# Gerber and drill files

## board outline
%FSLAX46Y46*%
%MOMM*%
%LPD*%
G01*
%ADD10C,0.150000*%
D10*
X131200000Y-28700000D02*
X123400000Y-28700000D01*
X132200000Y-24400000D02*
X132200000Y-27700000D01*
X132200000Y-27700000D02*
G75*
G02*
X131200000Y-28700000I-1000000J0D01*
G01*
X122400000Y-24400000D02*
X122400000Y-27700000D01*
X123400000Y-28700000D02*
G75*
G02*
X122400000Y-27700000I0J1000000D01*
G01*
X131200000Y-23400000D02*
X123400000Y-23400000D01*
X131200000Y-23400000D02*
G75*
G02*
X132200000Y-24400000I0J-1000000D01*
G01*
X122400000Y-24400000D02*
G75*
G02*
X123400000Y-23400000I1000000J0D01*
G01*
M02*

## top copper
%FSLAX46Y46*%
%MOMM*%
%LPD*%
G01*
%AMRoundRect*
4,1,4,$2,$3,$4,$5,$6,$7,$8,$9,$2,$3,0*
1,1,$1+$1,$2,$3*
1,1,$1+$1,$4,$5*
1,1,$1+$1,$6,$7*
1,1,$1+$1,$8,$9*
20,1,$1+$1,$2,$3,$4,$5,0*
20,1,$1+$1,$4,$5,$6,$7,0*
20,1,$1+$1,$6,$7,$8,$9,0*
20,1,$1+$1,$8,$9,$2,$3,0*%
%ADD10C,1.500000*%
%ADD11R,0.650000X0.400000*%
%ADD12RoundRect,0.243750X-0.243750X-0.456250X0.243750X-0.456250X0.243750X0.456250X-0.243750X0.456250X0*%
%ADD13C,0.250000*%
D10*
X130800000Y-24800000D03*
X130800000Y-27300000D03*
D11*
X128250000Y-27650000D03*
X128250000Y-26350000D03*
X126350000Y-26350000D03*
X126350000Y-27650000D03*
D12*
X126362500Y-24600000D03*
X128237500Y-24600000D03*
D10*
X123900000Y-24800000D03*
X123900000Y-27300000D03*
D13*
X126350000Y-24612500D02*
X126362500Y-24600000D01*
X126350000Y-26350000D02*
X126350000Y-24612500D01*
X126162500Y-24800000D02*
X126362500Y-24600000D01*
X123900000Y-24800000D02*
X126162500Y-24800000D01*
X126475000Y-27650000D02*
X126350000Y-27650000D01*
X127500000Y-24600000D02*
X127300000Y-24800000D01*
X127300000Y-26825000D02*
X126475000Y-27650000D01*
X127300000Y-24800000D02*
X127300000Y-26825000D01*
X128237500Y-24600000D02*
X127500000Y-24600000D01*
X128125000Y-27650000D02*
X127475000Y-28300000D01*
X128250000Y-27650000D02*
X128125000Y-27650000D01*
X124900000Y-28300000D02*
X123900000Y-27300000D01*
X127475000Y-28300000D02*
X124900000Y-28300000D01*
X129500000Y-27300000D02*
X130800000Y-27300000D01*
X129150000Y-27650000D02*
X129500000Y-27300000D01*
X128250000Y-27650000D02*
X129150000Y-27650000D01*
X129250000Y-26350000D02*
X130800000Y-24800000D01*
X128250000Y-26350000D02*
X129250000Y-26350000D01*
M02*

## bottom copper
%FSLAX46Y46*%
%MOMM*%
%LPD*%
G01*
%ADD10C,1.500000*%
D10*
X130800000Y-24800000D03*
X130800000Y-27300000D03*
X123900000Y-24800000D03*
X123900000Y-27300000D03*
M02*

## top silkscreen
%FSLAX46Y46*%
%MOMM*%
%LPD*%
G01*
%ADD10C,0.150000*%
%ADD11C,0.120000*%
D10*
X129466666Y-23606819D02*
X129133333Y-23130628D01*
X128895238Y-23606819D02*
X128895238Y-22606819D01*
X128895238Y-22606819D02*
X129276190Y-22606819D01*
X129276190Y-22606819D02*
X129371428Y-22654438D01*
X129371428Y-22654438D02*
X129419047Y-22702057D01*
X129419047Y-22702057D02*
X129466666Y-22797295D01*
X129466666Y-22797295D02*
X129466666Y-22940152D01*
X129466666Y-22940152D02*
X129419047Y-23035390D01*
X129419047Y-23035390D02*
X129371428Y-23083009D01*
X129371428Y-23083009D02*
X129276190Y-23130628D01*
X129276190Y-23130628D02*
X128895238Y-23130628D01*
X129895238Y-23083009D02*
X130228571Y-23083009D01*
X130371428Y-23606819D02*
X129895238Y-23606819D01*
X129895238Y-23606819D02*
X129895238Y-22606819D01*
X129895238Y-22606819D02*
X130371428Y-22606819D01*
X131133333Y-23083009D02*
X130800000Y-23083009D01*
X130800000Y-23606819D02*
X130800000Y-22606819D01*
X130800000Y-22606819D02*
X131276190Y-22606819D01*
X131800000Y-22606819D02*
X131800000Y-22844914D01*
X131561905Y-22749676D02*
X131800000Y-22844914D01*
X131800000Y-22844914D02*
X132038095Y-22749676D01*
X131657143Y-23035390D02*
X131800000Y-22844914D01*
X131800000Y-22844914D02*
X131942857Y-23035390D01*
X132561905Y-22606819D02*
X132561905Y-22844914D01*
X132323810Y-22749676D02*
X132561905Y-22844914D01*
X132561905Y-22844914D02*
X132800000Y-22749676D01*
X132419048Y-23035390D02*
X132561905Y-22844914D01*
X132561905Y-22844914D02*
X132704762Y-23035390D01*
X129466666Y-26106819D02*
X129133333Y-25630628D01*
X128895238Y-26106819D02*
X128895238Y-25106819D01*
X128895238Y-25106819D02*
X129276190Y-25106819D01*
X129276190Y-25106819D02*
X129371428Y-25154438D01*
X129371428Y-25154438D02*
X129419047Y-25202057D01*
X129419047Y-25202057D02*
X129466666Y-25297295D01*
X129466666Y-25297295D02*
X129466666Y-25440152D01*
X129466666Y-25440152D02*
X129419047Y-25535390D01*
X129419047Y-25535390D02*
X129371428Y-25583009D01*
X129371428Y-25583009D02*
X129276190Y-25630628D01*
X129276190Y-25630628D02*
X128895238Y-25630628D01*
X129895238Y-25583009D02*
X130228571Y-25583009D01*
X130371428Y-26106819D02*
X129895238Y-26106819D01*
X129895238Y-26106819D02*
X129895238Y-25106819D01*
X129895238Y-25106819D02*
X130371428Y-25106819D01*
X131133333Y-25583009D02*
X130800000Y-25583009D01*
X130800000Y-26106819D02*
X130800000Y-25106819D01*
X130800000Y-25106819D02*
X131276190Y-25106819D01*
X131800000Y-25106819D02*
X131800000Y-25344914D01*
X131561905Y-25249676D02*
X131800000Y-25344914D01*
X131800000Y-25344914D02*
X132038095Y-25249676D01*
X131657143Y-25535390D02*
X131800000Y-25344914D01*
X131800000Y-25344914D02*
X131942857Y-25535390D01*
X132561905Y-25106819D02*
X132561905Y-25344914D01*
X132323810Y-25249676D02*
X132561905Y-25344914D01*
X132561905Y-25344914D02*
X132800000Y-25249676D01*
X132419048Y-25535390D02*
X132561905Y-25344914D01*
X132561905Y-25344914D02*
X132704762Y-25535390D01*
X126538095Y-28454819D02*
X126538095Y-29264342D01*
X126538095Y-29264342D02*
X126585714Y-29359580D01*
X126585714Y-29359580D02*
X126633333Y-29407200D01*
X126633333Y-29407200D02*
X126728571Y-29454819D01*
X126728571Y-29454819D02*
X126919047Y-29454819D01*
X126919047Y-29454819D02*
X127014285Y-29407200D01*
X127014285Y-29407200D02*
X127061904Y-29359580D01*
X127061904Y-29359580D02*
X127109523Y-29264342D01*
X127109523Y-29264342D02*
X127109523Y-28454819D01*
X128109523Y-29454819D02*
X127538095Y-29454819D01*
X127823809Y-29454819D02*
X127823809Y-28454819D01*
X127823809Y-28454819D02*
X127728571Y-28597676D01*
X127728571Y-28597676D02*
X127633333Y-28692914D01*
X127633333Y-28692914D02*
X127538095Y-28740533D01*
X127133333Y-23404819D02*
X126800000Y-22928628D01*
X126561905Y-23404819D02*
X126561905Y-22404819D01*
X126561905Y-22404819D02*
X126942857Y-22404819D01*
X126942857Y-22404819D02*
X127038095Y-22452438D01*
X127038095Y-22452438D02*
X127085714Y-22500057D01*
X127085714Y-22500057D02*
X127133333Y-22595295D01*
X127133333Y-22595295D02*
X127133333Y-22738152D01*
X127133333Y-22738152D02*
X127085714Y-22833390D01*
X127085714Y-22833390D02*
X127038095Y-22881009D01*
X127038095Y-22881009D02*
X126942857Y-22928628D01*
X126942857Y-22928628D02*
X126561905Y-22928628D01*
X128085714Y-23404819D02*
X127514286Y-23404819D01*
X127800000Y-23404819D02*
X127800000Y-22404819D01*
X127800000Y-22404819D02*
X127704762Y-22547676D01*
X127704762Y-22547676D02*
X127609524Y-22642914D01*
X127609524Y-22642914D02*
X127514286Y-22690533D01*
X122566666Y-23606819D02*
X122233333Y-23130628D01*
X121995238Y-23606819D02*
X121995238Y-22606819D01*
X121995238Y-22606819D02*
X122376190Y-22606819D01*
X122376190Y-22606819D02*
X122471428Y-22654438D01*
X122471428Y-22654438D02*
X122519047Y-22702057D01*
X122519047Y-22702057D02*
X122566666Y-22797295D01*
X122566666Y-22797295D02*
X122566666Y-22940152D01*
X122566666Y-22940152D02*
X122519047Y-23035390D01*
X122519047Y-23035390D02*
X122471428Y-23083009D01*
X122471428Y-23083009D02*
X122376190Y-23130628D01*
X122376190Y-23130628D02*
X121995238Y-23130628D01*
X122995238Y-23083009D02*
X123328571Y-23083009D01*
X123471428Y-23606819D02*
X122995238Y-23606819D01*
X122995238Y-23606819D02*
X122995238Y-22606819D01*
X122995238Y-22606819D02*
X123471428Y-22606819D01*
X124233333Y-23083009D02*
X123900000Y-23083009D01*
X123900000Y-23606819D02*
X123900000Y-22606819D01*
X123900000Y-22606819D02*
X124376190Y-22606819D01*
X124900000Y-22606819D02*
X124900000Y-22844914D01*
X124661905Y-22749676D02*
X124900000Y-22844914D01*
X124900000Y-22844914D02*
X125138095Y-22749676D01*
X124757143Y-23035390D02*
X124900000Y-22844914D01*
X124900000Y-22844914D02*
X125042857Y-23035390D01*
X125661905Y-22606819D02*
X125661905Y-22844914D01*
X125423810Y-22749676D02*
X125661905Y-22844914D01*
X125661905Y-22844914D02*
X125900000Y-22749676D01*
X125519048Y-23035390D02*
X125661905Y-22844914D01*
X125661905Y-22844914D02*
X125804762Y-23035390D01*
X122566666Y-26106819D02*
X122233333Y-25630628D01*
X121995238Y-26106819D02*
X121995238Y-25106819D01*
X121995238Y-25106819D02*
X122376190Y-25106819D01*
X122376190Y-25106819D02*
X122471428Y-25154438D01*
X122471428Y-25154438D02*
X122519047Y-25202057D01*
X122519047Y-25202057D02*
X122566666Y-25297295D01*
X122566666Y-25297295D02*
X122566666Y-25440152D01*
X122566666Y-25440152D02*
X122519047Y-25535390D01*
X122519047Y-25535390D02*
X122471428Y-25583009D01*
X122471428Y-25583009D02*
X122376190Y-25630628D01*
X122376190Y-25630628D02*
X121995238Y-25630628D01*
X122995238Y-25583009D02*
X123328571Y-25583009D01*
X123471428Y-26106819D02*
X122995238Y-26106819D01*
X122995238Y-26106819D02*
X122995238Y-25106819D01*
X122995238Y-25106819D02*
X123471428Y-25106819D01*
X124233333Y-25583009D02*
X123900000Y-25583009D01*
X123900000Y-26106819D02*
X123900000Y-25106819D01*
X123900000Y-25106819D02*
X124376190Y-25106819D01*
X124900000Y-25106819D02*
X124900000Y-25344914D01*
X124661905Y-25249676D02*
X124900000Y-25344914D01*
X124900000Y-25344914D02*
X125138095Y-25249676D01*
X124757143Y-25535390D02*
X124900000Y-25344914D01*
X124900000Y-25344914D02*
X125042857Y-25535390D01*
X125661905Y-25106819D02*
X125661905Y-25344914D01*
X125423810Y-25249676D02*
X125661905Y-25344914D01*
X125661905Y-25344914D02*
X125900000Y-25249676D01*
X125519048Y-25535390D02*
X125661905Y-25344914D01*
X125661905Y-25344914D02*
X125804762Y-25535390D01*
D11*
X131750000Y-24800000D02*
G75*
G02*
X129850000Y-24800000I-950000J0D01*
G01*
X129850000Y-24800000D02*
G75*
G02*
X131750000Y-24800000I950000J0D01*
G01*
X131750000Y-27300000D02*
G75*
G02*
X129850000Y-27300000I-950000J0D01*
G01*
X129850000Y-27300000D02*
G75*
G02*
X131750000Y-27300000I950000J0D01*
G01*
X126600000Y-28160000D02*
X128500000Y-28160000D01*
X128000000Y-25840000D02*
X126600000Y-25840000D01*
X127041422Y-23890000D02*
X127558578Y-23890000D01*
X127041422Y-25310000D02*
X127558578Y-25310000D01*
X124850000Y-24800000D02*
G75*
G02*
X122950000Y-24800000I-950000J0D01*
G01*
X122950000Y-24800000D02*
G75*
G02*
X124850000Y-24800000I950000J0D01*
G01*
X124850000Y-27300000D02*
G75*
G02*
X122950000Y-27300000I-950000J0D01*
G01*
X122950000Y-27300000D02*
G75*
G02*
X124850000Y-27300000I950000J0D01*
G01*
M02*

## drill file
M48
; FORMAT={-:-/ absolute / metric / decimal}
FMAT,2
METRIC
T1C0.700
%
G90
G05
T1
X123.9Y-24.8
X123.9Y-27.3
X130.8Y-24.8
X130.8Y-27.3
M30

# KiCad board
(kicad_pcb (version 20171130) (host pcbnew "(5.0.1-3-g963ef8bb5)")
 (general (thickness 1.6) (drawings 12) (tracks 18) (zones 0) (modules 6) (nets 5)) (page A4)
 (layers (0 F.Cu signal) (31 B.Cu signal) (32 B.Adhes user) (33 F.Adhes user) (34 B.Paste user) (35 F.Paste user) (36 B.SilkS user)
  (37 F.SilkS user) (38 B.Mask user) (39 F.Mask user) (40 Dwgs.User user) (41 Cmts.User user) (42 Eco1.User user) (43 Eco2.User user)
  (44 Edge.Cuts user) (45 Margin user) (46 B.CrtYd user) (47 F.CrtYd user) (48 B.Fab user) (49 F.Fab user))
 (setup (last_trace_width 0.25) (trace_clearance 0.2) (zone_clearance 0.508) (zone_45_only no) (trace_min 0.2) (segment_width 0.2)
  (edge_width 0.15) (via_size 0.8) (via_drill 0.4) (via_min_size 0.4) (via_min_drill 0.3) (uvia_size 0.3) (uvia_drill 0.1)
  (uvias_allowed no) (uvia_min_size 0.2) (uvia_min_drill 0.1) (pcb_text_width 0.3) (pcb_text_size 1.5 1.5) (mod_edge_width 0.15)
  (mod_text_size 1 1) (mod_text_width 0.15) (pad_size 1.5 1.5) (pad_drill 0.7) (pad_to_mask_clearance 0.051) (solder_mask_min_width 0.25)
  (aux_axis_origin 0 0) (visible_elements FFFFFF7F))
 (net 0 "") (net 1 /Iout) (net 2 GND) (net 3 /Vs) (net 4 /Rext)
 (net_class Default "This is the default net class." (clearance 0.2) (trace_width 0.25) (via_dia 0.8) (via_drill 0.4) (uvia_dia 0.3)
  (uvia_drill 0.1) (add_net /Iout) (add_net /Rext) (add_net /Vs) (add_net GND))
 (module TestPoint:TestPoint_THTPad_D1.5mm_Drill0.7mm (layer F.Cu) (at 130.8 24.8)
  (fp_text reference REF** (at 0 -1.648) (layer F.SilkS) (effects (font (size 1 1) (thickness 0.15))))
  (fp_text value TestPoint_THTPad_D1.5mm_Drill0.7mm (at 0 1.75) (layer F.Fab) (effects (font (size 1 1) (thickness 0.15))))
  (fp_circle (center 0 0) (end 0 0.95) (layer F.SilkS) (width 0.12))
  (pad 1 thru_hole circle (at 0 0) (size 1.5 1.5) (drill 0.7) (layers *.Cu *.Mask) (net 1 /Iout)))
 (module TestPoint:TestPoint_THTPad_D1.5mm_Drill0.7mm (layer F.Cu) (at 130.8 27.3)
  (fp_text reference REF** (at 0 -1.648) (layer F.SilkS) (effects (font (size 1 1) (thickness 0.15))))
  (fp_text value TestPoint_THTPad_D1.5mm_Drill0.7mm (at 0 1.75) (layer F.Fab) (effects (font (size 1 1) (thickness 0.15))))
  (fp_circle (center 0 0) (end 0 0.95) (layer F.SilkS) (width 0.12))
  (pad 1 thru_hole circle (at 0 0) (size 1.5 1.5) (drill 0.7) (layers *.Cu *.Mask) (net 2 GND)))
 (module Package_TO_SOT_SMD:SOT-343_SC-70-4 (layer F.Cu) (at 127.3 27 180)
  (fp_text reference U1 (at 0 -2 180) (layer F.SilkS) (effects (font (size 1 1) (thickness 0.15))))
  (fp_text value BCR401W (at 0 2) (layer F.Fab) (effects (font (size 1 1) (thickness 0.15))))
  (fp_line (start 0.7 -1.16) (end -1.2 -1.16) (layer F.SilkS) (width 0.12))
  (fp_line (start -0.7 1.16) (end 0.7 1.16) (layer F.SilkS) (width 0.12))
  (pad 1 smd rect (at -0.95 -0.65 180) (size 0.65 0.4) (layers F.Cu F.Paste F.Mask) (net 2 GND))
  (pad 2 smd rect (at -0.95 0.65 180) (size 0.65 0.4) (layers F.Cu F.Paste F.Mask) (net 1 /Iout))
  (pad 3 smd rect (at 0.95 0.65 180) (size 0.65 0.4) (layers F.Cu F.Paste F.Mask) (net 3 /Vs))
  (pad 4 smd rect (at 0.95 -0.65 180) (size 0.65 0.4) (layers F.Cu F.Paste F.Mask) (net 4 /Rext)))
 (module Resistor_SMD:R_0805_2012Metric (layer F.Cu) (at 127.3 24.6)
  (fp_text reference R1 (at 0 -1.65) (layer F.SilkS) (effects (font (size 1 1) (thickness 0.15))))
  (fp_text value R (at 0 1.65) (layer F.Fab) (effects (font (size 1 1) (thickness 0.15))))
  (fp_line (start -0.258578 -0.71) (end 0.258578 -0.71) (layer F.SilkS) (width 0.12))
  (fp_line (start -0.258578 0.71) (end 0.258578 0.71) (layer F.SilkS) (width 0.12))
  (pad 1 smd roundrect (at -0.9375 0) (size 0.975 1.4) (layers F.Cu F.Paste F.Mask) (roundrect_rratio 0.25) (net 3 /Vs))
  (pad 2 smd roundrect (at 0.9375 0) (size 0.975 1.4) (layers F.Cu F.Paste F.Mask) (roundrect_rratio 0.25) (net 4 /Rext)))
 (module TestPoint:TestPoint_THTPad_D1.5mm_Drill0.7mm (layer F.Cu) (at 123.9 24.8)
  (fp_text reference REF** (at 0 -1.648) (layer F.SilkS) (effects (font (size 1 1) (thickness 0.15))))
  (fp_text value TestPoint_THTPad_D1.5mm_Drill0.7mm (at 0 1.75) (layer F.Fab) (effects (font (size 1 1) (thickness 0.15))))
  (fp_circle (center 0 0) (end 0 0.95) (layer F.SilkS) (width 0.12))
  (pad 1 thru_hole circle (at 0 0) (size 1.5 1.5) (drill 0.7) (layers *.Cu *.Mask) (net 3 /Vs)))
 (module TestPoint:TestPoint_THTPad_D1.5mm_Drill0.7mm (layer F.Cu) (at 123.9 27.3)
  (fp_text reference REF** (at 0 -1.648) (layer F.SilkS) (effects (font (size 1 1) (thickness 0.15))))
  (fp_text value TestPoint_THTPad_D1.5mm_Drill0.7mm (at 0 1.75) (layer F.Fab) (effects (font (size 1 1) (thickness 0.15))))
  (fp_circle (center 0 0) (end 0 0.95) (layer F.SilkS) (width 0.12))
  (pad 1 thru_hole circle (at 0 0) (size 1.5 1.5) (drill 0.7) (layers *.Cu *.Mask) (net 2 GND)))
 (gr_line (start 131.2 28.7) (end 123.4 28.7) (layer Edge.Cuts) (width 0.15))
 (gr_line (start 132.2 24.4) (end 132.2 27.7) (layer Edge.Cuts) (width 0.15))
 (gr_arc (start 131.2 27.7) (end 131.2 28.7) (angle -90) (layer Edge.Cuts) (width 0.15))
 (gr_line (start 122.4 24.4) (end 122.4 27.7) (layer Edge.Cuts) (width 0.15))
 (gr_arc (start 123.4 27.7) (end 122.4 27.7) (angle -90) (layer Edge.Cuts) (width 0.15))
 (gr_line (start 131.2 23.4) (end 123.4 23.4) (layer Edge.Cuts) (width 0.15))
 (gr_arc (start 131.2 24.4) (end 132.2 24.4) (angle -90) (layer Edge.Cuts) (width 0.15))
 (gr_arc (start 123.4 24.4) (end 123.4 23.4) (angle -90) (layer Edge.Cuts) (width 0.15))
 (segment (start 126.35 24.6125) (end 126.3625 24.6) (width 0.25) (layer F.Cu) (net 3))
 (segment (start 126.35 26.35) (end 126.35 24.6125) (width 0.25) (layer F.Cu) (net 3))
 (segment (start 126.1625 24.8) (end 126.3625 24.6) (width 0.25) (layer F.Cu) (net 3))
 (segment (start 123.9 24.8) (end 126.1625 24.8) (width 0.25) (layer F.Cu) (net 3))
 (segment (start 126.475 27.65) (end 126.35 27.65) (width 0.25) (layer F.Cu) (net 4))
 (segment (start 127.5 24.6) (end 127.3 24.8) (width 0.25) (layer F.Cu) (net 4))
 (segment (start 127.3 26.825) (end 126.475 27.65) (width 0.25) (layer F.Cu) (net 4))
 (segment (start 127.3 24.8) (end 127.3 26.825) (width 0.25) (layer F.Cu) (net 4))
 (segment (start 128.2375 24.6) (end 127.5 24.6) (width 0.25) (layer F.Cu) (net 4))
 (segment (start 128.125 27.65) (end 127.475 28.3) (width 0.25) (layer F.Cu) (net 2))
 (segment (start 128.25 27.65) (end 128.125 27.65) (width 0.25) (layer F.Cu) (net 2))
 (segment (start 124.9 28.3) (end 123.9 27.3) (width 0.25) (layer F.Cu) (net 2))
 (segment (start 127.475 28.3) (end 124.9 28.3) (width 0.25) (layer F.Cu) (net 2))
 (segment (start 129.5 27.3) (end 130.8 27.3) (width 0.25) (layer F.Cu) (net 2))
 (segment (start 129.15 27.65) (end 129.5 27.3) (width 0.25) (layer F.Cu) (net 2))
 (segment (start 128.25 27.65) (end 129.15 27.65) (width 0.25) (layer F.Cu) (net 2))
 (segment (start 129.25 26.35) (end 130.8 24.8) (width 0.25) (layer F.Cu) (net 1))
 (segment (start 128.25 26.35) (end 129.25 26.35) (width 0.25) (layer F.Cu) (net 1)))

